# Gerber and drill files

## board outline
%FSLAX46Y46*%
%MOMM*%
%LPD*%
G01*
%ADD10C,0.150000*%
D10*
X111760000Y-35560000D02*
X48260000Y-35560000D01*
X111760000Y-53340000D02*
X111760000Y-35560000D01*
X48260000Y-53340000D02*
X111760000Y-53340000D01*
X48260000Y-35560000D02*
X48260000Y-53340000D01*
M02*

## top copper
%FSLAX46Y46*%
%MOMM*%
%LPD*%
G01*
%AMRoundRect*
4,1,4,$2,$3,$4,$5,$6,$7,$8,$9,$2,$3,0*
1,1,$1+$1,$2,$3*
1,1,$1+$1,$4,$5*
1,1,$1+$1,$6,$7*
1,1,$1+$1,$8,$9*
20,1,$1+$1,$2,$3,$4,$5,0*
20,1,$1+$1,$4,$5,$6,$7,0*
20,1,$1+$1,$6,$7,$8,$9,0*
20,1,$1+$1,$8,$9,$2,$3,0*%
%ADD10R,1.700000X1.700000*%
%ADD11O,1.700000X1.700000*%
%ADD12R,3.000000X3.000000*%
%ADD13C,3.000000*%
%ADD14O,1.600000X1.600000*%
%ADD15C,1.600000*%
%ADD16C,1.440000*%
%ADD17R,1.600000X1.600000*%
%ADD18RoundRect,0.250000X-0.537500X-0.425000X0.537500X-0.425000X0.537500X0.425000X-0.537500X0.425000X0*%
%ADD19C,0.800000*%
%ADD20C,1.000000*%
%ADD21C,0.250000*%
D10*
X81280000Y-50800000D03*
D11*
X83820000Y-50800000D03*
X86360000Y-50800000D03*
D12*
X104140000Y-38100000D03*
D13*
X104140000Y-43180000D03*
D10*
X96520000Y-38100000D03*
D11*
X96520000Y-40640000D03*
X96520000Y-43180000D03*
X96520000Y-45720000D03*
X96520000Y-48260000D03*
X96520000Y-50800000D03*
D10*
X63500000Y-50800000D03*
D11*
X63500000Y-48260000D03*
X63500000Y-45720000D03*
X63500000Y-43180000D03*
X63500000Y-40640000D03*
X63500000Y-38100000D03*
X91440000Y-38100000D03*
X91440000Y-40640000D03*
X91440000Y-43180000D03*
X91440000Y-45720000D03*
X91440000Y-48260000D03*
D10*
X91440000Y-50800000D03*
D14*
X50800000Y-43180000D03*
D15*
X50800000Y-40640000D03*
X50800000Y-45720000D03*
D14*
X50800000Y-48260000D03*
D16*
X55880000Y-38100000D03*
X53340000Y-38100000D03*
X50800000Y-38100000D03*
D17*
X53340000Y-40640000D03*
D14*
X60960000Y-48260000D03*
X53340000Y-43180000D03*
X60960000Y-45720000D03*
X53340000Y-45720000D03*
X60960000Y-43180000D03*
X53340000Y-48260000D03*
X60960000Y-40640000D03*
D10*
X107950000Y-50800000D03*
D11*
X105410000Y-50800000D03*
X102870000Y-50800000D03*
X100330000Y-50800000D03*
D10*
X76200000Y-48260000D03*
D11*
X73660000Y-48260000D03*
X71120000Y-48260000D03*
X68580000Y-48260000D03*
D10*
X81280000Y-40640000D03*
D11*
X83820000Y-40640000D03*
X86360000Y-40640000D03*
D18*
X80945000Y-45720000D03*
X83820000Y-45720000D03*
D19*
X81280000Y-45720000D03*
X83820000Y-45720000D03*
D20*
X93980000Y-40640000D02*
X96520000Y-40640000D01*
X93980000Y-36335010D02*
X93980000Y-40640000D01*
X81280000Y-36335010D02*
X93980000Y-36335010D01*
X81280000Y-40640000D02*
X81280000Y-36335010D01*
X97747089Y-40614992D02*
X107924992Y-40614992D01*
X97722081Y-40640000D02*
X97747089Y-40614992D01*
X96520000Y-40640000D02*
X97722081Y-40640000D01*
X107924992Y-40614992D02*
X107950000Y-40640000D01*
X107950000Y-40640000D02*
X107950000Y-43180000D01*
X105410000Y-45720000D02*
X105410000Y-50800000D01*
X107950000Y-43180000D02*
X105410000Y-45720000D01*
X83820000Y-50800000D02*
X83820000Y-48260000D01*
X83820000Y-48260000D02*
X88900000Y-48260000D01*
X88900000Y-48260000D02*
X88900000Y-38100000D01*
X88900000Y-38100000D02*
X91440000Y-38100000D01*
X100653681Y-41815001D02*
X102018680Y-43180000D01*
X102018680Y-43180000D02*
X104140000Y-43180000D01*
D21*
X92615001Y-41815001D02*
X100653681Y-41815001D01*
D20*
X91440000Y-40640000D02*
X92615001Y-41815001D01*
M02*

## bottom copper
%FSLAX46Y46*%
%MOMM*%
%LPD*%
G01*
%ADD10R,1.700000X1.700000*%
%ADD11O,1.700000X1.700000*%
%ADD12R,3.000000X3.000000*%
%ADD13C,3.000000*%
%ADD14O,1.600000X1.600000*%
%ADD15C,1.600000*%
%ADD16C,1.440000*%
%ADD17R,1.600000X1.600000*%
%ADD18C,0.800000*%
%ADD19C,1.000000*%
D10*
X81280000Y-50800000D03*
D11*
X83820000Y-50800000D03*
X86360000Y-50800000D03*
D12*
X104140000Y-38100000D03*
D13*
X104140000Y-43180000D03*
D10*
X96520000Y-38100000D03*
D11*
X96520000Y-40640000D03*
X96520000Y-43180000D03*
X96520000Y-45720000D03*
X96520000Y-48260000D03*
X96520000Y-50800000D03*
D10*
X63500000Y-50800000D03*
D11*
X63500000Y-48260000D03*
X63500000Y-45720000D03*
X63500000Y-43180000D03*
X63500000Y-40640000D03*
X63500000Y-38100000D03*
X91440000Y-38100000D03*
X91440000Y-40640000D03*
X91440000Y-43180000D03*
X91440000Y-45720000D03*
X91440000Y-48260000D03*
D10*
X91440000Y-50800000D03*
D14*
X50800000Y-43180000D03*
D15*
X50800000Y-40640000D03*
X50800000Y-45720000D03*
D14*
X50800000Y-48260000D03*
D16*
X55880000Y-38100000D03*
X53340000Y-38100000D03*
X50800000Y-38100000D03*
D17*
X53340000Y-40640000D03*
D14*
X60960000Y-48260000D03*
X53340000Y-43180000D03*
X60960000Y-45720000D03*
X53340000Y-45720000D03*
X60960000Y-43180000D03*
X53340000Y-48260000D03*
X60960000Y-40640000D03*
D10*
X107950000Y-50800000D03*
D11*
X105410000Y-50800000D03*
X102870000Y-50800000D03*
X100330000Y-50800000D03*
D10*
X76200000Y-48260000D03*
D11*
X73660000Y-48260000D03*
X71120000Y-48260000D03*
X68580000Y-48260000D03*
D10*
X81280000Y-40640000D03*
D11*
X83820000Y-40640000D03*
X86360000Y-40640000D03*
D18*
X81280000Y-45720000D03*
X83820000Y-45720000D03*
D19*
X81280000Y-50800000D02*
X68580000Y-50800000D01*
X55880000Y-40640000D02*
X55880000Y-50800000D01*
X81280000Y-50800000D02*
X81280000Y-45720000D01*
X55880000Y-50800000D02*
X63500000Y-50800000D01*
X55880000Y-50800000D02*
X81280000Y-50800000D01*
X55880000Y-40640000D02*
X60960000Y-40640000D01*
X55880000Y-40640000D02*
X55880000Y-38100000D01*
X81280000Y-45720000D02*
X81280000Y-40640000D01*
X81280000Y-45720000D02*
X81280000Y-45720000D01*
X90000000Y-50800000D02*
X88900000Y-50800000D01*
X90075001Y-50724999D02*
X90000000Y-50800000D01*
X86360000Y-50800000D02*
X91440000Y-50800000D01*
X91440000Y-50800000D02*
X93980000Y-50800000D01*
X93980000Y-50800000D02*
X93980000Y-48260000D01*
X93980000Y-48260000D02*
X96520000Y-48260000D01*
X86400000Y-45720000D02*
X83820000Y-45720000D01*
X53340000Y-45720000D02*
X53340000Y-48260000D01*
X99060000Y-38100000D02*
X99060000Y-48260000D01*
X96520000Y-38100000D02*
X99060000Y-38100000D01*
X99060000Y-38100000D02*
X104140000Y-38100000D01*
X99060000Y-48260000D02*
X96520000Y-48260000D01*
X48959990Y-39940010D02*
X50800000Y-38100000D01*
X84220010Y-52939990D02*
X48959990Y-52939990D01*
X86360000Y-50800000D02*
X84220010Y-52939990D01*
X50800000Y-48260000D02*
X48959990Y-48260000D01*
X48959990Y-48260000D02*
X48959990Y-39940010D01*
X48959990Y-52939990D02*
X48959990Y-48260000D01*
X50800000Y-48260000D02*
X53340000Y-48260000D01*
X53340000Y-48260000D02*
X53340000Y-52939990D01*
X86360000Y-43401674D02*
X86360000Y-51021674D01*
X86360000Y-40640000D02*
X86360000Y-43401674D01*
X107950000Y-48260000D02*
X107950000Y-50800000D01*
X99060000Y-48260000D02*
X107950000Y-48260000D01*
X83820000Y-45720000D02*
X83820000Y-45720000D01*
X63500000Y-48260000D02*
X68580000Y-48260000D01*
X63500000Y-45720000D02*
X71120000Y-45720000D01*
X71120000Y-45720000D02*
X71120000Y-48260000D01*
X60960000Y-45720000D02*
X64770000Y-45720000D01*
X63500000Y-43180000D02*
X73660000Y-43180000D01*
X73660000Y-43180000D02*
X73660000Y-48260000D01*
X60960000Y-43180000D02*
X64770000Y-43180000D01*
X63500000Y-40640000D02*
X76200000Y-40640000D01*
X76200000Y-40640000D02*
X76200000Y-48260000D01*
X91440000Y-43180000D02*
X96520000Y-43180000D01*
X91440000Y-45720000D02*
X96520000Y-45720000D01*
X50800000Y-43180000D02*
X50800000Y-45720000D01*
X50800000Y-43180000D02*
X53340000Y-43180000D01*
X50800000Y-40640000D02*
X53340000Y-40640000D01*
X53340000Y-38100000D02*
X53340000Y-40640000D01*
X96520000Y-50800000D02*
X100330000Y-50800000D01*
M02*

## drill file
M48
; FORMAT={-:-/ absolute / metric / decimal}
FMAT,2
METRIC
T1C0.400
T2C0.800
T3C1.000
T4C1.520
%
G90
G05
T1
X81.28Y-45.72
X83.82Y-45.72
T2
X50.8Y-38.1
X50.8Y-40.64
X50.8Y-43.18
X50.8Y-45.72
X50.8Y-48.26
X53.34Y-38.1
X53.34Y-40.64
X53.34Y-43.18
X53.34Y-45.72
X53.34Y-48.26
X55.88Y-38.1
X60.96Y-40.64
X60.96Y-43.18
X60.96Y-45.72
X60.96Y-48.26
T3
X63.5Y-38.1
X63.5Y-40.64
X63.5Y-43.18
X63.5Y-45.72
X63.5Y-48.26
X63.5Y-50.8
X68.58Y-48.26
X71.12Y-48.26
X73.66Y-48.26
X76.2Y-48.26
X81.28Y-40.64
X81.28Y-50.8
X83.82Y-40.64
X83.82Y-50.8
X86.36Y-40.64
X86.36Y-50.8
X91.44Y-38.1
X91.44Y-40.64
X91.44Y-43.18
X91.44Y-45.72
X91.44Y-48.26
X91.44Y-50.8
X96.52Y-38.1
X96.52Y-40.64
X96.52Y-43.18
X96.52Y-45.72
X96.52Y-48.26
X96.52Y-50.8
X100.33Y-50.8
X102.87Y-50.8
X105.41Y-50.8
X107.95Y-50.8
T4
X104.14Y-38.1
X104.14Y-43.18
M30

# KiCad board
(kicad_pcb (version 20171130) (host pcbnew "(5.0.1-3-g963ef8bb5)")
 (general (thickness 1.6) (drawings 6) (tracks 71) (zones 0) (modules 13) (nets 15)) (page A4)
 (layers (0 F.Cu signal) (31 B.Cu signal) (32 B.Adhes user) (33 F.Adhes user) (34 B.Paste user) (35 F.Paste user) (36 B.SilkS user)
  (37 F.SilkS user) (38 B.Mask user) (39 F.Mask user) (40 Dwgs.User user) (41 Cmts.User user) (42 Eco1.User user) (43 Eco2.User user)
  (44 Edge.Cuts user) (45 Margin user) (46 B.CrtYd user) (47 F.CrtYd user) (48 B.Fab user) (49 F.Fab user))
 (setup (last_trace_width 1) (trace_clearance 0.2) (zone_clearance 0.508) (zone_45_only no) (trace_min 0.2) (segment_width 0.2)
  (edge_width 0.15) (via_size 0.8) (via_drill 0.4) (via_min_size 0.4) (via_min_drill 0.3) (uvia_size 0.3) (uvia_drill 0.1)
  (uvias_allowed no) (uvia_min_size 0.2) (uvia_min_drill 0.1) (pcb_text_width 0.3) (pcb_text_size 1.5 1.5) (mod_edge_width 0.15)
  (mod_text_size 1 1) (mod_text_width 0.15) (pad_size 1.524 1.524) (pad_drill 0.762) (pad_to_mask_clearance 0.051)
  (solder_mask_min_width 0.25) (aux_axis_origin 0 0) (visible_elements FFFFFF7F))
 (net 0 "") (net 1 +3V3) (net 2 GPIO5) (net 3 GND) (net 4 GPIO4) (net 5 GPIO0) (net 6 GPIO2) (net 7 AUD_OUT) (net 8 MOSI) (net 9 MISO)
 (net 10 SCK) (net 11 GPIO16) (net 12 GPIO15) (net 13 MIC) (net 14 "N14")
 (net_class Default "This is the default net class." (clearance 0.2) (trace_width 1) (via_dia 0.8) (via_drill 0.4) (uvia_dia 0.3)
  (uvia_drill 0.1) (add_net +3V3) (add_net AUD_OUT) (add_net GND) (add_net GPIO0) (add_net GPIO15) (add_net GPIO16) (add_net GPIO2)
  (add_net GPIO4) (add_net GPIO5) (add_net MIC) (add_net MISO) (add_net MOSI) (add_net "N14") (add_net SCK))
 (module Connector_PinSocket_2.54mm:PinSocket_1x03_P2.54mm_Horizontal (layer F.Cu) (at 81.28 50.8 90)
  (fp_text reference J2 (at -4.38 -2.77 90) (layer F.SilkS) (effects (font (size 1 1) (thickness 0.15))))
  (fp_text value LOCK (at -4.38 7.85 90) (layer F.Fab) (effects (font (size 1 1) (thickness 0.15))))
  (pad 1 thru_hole rect (at 0 0 90) (size 1.7 1.7) (drill 1) (layers *.Cu *.Mask) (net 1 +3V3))
  (pad 2 thru_hole oval (at 0 2.54 90) (size 1.7 1.7) (drill 1) (layers *.Cu *.Mask) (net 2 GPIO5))
  (pad 3 thru_hole oval (at 0 5.08 90) (size 1.7 1.7) (drill 1) (layers *.Cu *.Mask) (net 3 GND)))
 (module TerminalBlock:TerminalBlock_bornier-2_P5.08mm (layer F.Cu) (at 104.14 38.1 270)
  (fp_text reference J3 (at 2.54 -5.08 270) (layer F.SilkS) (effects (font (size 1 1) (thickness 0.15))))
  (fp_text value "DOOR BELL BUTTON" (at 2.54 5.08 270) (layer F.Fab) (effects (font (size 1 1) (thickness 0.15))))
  (pad 1 thru_hole rect (at 0 0 270) (size 3 3) (drill 1.52) (layers *.Cu *.Mask) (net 3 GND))
  (pad 2 thru_hole circle (at 5.08 0 270) (size 3 3) (drill 1.52) (layers *.Cu *.Mask) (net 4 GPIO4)))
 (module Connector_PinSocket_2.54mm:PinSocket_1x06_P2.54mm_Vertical (layer F.Cu) (at 96.52 38.1)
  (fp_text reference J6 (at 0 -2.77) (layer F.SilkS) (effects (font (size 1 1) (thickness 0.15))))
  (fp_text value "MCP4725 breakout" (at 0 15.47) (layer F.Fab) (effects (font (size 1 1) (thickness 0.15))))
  (pad 1 thru_hole rect (at 0 0) (size 1.7 1.7) (drill 1) (layers *.Cu *.Mask) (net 3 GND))
  (pad 2 thru_hole oval (at 0 2.54) (size 1.7 1.7) (drill 1) (layers *.Cu *.Mask) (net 1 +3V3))
  (pad 3 thru_hole oval (at 0 5.08) (size 1.7 1.7) (drill 1) (layers *.Cu *.Mask) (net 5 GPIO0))
  (pad 4 thru_hole oval (at 0 7.62) (size 1.7 1.7) (drill 1) (layers *.Cu *.Mask) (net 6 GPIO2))
  (pad 5 thru_hole oval (at 0 10.16) (size 1.7 1.7) (drill 1) (layers *.Cu *.Mask) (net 3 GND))
  (pad 6 thru_hole oval (at 0 12.7) (size 1.7 1.7) (drill 1) (layers *.Cu *.Mask) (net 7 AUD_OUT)))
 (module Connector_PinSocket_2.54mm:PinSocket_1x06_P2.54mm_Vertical (layer F.Cu) (at 63.5 50.8 180)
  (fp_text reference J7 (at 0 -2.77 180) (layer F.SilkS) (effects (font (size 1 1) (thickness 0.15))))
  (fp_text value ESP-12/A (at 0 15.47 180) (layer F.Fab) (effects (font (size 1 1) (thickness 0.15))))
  (pad 1 thru_hole rect (at 0 0 180) (size 1.7 1.7) (drill 1) (layers *.Cu *.Mask) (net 1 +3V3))
  (pad 2 thru_hole oval (at 0 2.54 180) (size 1.7 1.7) (drill 1) (layers *.Cu *.Mask) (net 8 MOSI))
  (pad 3 thru_hole oval (at 0 5.08 180) (size 1.7 1.7) (drill 1) (layers *.Cu *.Mask) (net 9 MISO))
  (pad 4 thru_hole oval (at 0 7.62 180) (size 1.7 1.7) (drill 1) (layers *.Cu *.Mask) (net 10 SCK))
  (pad 5 thru_hole oval (at 0 10.16 180) (size 1.7 1.7) (drill 1) (layers *.Cu *.Mask) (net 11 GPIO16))
  (pad 6 thru_hole oval (at 0 12.7 180) (size 1.7 1.7) (drill 1) (layers *.Cu *.Mask)))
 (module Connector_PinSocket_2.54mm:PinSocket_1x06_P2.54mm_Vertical (layer F.Cu) (at 91.44 50.8 180)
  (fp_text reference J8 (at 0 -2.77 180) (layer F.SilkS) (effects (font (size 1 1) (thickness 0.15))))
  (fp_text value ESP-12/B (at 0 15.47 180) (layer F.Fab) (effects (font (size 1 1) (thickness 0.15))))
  (pad 6 thru_hole oval (at 0 12.7 180) (size 1.7 1.7) (drill 1) (layers *.Cu *.Mask) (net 2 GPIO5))
  (pad 5 thru_hole oval (at 0 10.16 180) (size 1.7 1.7) (drill 1) (layers *.Cu *.Mask) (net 4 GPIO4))
  (pad 4 thru_hole oval (at 0 7.62 180) (size 1.7 1.7) (drill 1) (layers *.Cu *.Mask) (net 5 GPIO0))
  (pad 3 thru_hole oval (at 0 5.08 180) (size 1.7 1.7) (drill 1) (layers *.Cu *.Mask) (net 6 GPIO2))
  (pad 2 thru_hole oval (at 0 2.54 180) (size 1.7 1.7) (drill 1) (layers *.Cu *.Mask) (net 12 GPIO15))
  (pad 1 thru_hole rect (at 0 0 180) (size 1.7 1.7) (drill 1) (layers *.Cu *.Mask) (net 3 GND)))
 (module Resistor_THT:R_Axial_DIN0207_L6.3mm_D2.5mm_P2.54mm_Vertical (layer F.Cu) (at 50.8 40.64 270)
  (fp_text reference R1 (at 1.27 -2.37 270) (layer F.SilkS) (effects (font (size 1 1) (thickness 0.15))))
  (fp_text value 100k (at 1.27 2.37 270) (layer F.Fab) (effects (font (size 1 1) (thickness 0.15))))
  (pad 2 thru_hole oval (at 2.54 0 270) (size 1.6 1.6) (drill 0.8) (layers *.Cu *.Mask) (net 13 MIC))
  (pad 1 thru_hole circle (at 0 0 270) (size 1.6 1.6) (drill 0.8) (layers *.Cu *.Mask) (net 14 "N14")))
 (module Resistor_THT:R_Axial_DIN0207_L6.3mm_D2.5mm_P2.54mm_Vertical (layer F.Cu) (at 50.8 45.72 270)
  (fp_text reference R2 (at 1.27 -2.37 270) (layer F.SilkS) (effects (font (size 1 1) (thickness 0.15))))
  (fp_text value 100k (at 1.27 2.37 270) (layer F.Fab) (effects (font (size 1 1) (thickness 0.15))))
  (pad 1 thru_hole circle (at 0 0 270) (size 1.6 1.6) (drill 0.8) (layers *.Cu *.Mask) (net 13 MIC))
  (pad 2 thru_hole oval (at 2.54 0 270) (size 1.6 1.6) (drill 0.8) (layers *.Cu *.Mask) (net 3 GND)))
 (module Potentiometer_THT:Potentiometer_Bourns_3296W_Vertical (layer F.Cu) (at 55.88 38.1)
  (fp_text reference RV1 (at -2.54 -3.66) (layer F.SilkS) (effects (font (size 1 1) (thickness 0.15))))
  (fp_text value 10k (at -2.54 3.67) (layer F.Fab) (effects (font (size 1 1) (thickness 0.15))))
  (pad 1 thru_hole circle (at 0 0) (size 1.44 1.44) (drill 0.8) (layers *.Cu *.Mask) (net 1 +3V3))
  (pad 2 thru_hole circle (at -2.54 0) (size 1.44 1.44) (drill 0.8) (layers *.Cu *.Mask) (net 14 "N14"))
  (pad 3 thru_hole circle (at -5.08 0) (size 1.44 1.44) (drill 0.8) (layers *.Cu *.Mask) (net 3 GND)))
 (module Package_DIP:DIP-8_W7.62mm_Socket (layer F.Cu) (at 53.34 40.64)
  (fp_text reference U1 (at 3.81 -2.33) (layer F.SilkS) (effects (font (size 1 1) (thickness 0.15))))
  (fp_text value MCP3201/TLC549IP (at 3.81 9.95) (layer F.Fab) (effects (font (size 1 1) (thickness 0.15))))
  (pad 1 thru_hole rect (at 0 0) (size 1.6 1.6) (drill 0.8) (layers *.Cu *.Mask) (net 14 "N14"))
  (pad 5 thru_hole oval (at 7.62 7.62) (size 1.6 1.6) (drill 0.8) (layers *.Cu *.Mask) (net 12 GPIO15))
  (pad 2 thru_hole oval (at 0 2.54) (size 1.6 1.6) (drill 0.8) (layers *.Cu *.Mask) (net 13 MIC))
  (pad 6 thru_hole oval (at 7.62 5.08) (size 1.6 1.6) (drill 0.8) (layers *.Cu *.Mask) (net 9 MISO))
  (pad 3 thru_hole oval (at 0 5.08) (size 1.6 1.6) (drill 0.8) (layers *.Cu *.Mask) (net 3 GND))
  (pad 7 thru_hole oval (at 7.62 2.54) (size 1.6 1.6) (drill 0.8) (layers *.Cu *.Mask) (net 10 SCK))
  (pad 4 thru_hole oval (at 0 7.62) (size 1.6 1.6) (drill 0.8) (layers *.Cu *.Mask) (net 3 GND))
  (pad 8 thru_hole oval (at 7.62 0) (size 1.6 1.6) (drill 0.8) (layers *.Cu *.Mask) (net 1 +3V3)))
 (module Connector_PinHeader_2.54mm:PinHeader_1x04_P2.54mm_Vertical (layer F.Cu) (at 107.95 50.8 270)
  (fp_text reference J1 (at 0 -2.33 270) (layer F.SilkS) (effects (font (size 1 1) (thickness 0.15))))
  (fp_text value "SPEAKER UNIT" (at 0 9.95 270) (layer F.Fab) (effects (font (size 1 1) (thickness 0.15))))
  (pad 1 thru_hole rect (at 0 0 270) (size 1.7 1.7) (drill 1) (layers *.Cu *.Mask) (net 3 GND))
  (pad 2 thru_hole oval (at 0 2.54 270) (size 1.7 1.7) (drill 1) (layers *.Cu *.Mask) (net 1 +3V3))
  (pad 3 thru_hole oval (at 0 5.08 270) (size 1.7 1.7) (drill 1) (layers *.Cu *.Mask) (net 13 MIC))
  (pad 4 thru_hole oval (at 0 7.62 270) (size 1.7 1.7) (drill 1) (layers *.Cu *.Mask) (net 7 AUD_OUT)))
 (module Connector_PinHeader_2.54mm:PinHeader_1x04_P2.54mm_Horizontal (layer F.Cu) (at 76.2 48.26 270)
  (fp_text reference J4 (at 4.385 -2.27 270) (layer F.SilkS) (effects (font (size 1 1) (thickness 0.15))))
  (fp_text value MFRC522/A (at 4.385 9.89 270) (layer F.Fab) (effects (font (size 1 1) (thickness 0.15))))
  (pad 1 thru_hole rect (at 0 0 270) (size 1.7 1.7) (drill 1) (layers *.Cu *.Mask) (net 11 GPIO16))
  (pad 2 thru_hole oval (at 0 2.54 270) (size 1.7 1.7) (drill 1) (layers *.Cu *.Mask) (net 10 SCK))
  (pad 3 thru_hole oval (at 0 5.08 270) (size 1.7 1.7) (drill 1) (layers *.Cu *.Mask) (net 9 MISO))
  (pad 4 thru_hole oval (at 0 7.62 270) (size 1.7 1.7) (drill 1) (layers *.Cu *.Mask) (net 8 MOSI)))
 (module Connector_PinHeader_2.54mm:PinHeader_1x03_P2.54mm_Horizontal (layer F.Cu) (at 81.28 40.64 90)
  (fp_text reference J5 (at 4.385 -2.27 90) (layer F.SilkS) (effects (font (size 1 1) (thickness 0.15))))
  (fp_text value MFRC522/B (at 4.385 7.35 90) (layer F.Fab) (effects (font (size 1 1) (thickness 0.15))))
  (pad 1 thru_hole rect (at 0 0 90) (size 1.7 1.7) (drill 1) (layers *.Cu *.Mask) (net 1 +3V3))
  (pad 2 thru_hole oval (at 0 2.54 90) (size 1.7 1.7) (drill 1) (layers *.Cu *.Mask) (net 4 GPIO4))
  (pad 3 thru_hole oval (at 0 5.08 90) (size 1.7 1.7) (drill 1) (layers *.Cu *.Mask) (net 3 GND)))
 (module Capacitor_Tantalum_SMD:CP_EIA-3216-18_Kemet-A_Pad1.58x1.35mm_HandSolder (layer F.Cu) (at 82.3825 45.72)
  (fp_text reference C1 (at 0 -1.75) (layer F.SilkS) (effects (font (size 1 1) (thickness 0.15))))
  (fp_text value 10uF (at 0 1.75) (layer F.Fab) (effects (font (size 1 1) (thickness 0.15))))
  (pad 1 smd roundrect (at -1.4375 0) (size 1.575 1.35) (layers F.Cu F.Paste F.Mask) (roundrect_rratio 0.185185) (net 1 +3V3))
  (pad 2 smd roundrect (at 1.4375 0) (size 1.575 1.35) (layers F.Cu F.Paste F.Mask) (roundrect_rratio 0.185185) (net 3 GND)))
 (gr_line (start 111.76 35.56) (end 48.26 35.56) (layer Edge.Cuts) (width 0.15))
 (gr_line (start 111.76 53.34) (end 111.76 35.56) (layer Edge.Cuts) (width 0.15))
 (gr_line (start 48.26 53.34) (end 111.76 53.34) (layer Edge.Cuts) (width 0.15))
 (gr_line (start 48.26 35.56) (end 48.26 53.34) (layer Edge.Cuts) (width 0.15))
 (segment (start 81.28 50.8) (end 68.58 50.8) (width 1) (layer B.Cu) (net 1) (status 10))
 (segment (start 55.88 40.64) (end 55.88 50.8) (width 1) (layer B.Cu) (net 1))
 (segment (start 81.28 50.8) (end 81.28 45.72) (width 1) (layer B.Cu) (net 1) (status 30))
 (segment (start 55.88 50.8) (end 63.5 50.8) (width 1) (layer B.Cu) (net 1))
 (segment (start 55.88 50.8) (end 81.28 50.8) (width 1) (layer B.Cu) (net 1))
 (segment (start 55.88 40.64) (end 60.96 40.64) (width 1) (layer B.Cu) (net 1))
 (segment (start 55.88 40.64) (end 55.88 38.1) (width 1) (layer B.Cu) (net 1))
 (segment (start 81.28 45.72) (end 81.28 40.64) (width 1) (layer B.Cu) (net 1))
 (segment (start 93.98 40.64) (end 96.52 40.64) (width 1) (layer F.Cu) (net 1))
 (segment (start 93.98 36.33501) (end 93.98 40.64) (width 1) (layer F.Cu) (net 1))
 (segment (start 81.28 36.33501) (end 93.98 36.33501) (width 1) (layer F.Cu) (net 1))
 (segment (start 81.28 40.64) (end 81.28 36.33501) (width 1) (layer F.Cu) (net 1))
 (segment (start 97.747089 40.614992) (end 107.924992 40.614992) (width 1) (layer F.Cu) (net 1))
 (segment (start 97.722081 40.64) (end 97.747089 40.614992) (width 1) (layer F.Cu) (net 1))
 (segment (start 96.52 40.64) (end 97.722081 40.64) (width 1) (layer F.Cu) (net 1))
 (segment (start 107.924992 40.614992) (end 107.95 40.64) (width 1) (layer F.Cu) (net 1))
 (segment (start 107.95 40.64) (end 107.95 43.18) (width 1) (layer F.Cu) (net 1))
 (segment (start 105.41 45.72) (end 105.41 50.8) (width 1) (layer F.Cu) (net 1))
 (segment (start 107.95 43.18) (end 105.41 45.72) (width 1) (layer F.Cu) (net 1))
 (segment (start 81.28 45.72) (end 81.28 45.72) (width 1) (layer B.Cu) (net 1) (status 30))
 (via (at 81.28 45.72) (size 0.8) (drill 0.4) (layers F.Cu B.Cu) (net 1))
 (segment (start 90 50.8) (end 88.9 50.8) (width 1) (layer B.Cu) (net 3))
 (segment (start 90.075001 50.724999) (end 90 50.8) (width 1) (layer B.Cu) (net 3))
 (segment (start 86.36 50.8) (end 91.44 50.8) (width 1) (layer B.Cu) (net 3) (status 30))
 (segment (start 91.44 50.8) (end 93.98 50.8) (width 1) (layer B.Cu) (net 3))
 (segment (start 93.98 50.8) (end 93.98 48.26) (width 1) (layer B.Cu) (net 3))
 (segment (start 93.98 48.26) (end 96.52 48.26) (width 1) (layer B.Cu) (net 3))
 (segment (start 86.4 45.72) (end 83.82 45.72) (width 1) (layer B.Cu) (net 3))
 (segment (start 53.34 45.72) (end 53.34 48.26) (width 1) (layer B.Cu) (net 3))
 (segment (start 99.06 38.1) (end 99.06 48.26) (width 1) (layer B.Cu) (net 3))
 (segment (start 96.52 38.1) (end 99.06 38.1) (width 1) (layer B.Cu) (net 3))
 (segment (start 99.06 38.1) (end 104.14 38.1) (width 1) (layer B.Cu) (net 3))
 (segment (start 99.06 48.26) (end 96.52 48.26) (width 1) (layer B.Cu) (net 3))
 (segment (start 48.95999 39.94001) (end 50.8 38.1) (width 1) (layer B.Cu) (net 3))
 (segment (start 84.22001 52.93999) (end 48.95999 52.93999) (width 1) (layer B.Cu) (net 3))
 (segment (start 86.36 50.8) (end 84.22001 52.93999) (width 1) (layer B.Cu) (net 3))
 (segment (start 50.8 48.26) (end 48.95999 48.26) (width 1) (layer B.Cu) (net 3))
 (segment (start 48.95999 48.26) (end 48.95999 39.94001) (width 1) (layer B.Cu) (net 3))
 (segment (start 48.95999 52.93999) (end 48.95999 48.26) (width 1) (layer B.Cu) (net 3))
 (segment (start 50.8 48.26) (end 53.34 48.26) (width 1) (layer B.Cu) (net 3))
 (segment (start 53.34 48.26) (end 53.34 52.93999) (width 1) (layer B.Cu) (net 3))
 (segment (start 86.36 43.401674) (end 86.36 51.021674) (width 1) (layer B.Cu) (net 3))
 (segment (start 86.36 40.64) (end 86.36 43.401674) (width 1) (layer B.Cu) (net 3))
 (segment (start 107.95 48.26) (end 107.95 50.8) (width 1) (layer B.Cu) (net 3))
 (segment (start 99.06 48.26) (end 107.95 48.26) (width 1) (layer B.Cu) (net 3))
 (segment (start 83.82 45.72) (end 83.82 45.72) (width 1) (layer B.Cu) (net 3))
 (via (at 83.82 45.72) (size 0.8) (drill 0.4) (layers F.Cu B.Cu) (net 3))
 (segment (start 83.82 50.8) (end 83.82 48.26) (width 1) (layer F.Cu) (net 2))
 (segment (start 83.82 48.26) (end 88.9 48.26) (width 1) (layer F.Cu) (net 2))
 (segment (start 88.9 48.26) (end 88.9 38.1) (width 1) (layer F.Cu) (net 2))
 (segment (start 88.9 38.1) (end 91.44 38.1) (width 1) (layer F.Cu) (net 2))
 (segment (start 100.653681 41.815001) (end 102.01868 43.18) (width 1) (layer F.Cu) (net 4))
 (segment (start 102.01868 43.18) (end 104.14 43.18) (width 1) (layer F.Cu) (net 4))
 (segment (start 92.615001 41.815001) (end 100.653681 41.815001) (width 0.25) (layer F.Cu) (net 4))
 (segment (start 91.44 40.64) (end 92.615001 41.815001) (width 1) (layer F.Cu) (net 4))
 (segment (start 63.5 48.26) (end 68.58 48.26) (width 1) (layer B.Cu) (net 8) (status 30))
 (segment (start 63.5 45.72) (end 71.12 45.72) (width 1) (layer B.Cu) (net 9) (status 10))
 (segment (start 71.12 45.72) (end 71.12 48.26) (width 1) (layer B.Cu) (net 9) (status 20))
 (segment (start 60.96 45.72) (end 64.77 45.72) (width 1) (layer B.Cu) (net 9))
 (segment (start 63.5 43.18) (end 73.66 43.18) (width 1) (layer B.Cu) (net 10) (status 10))
 (segment (start 73.66 43.18) (end 73.66 48.26) (width 1) (layer B.Cu) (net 10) (status 20))
 (segment (start 60.96 43.18) (end 64.77 43.18) (width 1) (layer B.Cu) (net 10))
 (segment (start 63.5 40.64) (end 76.2 40.64) (width 1) (layer B.Cu) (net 11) (status 10))
 (segment (start 76.2 40.64) (end 76.2 48.26) (width 1) (layer B.Cu) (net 11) (status 20))
 (segment (start 91.44 43.18) (end 96.52 43.18) (width 1) (layer B.Cu) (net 5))
 (segment (start 91.44 45.72) (end 96.52 45.72) (width 1) (layer B.Cu) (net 6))
 (segment (start 50.8 43.18) (end 50.8 45.72) (width 1) (layer B.Cu) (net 13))
 (segment (start 50.8 43.18) (end 53.34 43.18) (width 1) (layer B.Cu) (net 13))
 (segment (start 50.8 40.64) (end 53.34 40.64) (width 1) (layer B.Cu) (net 14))
 (segment (start 53.34 38.1) (end 53.34 40.64) (width 1) (layer B.Cu) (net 14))
 (segment (start 96.52 50.8) (end 100.33 50.8) (width 1) (layer B.Cu) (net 7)))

